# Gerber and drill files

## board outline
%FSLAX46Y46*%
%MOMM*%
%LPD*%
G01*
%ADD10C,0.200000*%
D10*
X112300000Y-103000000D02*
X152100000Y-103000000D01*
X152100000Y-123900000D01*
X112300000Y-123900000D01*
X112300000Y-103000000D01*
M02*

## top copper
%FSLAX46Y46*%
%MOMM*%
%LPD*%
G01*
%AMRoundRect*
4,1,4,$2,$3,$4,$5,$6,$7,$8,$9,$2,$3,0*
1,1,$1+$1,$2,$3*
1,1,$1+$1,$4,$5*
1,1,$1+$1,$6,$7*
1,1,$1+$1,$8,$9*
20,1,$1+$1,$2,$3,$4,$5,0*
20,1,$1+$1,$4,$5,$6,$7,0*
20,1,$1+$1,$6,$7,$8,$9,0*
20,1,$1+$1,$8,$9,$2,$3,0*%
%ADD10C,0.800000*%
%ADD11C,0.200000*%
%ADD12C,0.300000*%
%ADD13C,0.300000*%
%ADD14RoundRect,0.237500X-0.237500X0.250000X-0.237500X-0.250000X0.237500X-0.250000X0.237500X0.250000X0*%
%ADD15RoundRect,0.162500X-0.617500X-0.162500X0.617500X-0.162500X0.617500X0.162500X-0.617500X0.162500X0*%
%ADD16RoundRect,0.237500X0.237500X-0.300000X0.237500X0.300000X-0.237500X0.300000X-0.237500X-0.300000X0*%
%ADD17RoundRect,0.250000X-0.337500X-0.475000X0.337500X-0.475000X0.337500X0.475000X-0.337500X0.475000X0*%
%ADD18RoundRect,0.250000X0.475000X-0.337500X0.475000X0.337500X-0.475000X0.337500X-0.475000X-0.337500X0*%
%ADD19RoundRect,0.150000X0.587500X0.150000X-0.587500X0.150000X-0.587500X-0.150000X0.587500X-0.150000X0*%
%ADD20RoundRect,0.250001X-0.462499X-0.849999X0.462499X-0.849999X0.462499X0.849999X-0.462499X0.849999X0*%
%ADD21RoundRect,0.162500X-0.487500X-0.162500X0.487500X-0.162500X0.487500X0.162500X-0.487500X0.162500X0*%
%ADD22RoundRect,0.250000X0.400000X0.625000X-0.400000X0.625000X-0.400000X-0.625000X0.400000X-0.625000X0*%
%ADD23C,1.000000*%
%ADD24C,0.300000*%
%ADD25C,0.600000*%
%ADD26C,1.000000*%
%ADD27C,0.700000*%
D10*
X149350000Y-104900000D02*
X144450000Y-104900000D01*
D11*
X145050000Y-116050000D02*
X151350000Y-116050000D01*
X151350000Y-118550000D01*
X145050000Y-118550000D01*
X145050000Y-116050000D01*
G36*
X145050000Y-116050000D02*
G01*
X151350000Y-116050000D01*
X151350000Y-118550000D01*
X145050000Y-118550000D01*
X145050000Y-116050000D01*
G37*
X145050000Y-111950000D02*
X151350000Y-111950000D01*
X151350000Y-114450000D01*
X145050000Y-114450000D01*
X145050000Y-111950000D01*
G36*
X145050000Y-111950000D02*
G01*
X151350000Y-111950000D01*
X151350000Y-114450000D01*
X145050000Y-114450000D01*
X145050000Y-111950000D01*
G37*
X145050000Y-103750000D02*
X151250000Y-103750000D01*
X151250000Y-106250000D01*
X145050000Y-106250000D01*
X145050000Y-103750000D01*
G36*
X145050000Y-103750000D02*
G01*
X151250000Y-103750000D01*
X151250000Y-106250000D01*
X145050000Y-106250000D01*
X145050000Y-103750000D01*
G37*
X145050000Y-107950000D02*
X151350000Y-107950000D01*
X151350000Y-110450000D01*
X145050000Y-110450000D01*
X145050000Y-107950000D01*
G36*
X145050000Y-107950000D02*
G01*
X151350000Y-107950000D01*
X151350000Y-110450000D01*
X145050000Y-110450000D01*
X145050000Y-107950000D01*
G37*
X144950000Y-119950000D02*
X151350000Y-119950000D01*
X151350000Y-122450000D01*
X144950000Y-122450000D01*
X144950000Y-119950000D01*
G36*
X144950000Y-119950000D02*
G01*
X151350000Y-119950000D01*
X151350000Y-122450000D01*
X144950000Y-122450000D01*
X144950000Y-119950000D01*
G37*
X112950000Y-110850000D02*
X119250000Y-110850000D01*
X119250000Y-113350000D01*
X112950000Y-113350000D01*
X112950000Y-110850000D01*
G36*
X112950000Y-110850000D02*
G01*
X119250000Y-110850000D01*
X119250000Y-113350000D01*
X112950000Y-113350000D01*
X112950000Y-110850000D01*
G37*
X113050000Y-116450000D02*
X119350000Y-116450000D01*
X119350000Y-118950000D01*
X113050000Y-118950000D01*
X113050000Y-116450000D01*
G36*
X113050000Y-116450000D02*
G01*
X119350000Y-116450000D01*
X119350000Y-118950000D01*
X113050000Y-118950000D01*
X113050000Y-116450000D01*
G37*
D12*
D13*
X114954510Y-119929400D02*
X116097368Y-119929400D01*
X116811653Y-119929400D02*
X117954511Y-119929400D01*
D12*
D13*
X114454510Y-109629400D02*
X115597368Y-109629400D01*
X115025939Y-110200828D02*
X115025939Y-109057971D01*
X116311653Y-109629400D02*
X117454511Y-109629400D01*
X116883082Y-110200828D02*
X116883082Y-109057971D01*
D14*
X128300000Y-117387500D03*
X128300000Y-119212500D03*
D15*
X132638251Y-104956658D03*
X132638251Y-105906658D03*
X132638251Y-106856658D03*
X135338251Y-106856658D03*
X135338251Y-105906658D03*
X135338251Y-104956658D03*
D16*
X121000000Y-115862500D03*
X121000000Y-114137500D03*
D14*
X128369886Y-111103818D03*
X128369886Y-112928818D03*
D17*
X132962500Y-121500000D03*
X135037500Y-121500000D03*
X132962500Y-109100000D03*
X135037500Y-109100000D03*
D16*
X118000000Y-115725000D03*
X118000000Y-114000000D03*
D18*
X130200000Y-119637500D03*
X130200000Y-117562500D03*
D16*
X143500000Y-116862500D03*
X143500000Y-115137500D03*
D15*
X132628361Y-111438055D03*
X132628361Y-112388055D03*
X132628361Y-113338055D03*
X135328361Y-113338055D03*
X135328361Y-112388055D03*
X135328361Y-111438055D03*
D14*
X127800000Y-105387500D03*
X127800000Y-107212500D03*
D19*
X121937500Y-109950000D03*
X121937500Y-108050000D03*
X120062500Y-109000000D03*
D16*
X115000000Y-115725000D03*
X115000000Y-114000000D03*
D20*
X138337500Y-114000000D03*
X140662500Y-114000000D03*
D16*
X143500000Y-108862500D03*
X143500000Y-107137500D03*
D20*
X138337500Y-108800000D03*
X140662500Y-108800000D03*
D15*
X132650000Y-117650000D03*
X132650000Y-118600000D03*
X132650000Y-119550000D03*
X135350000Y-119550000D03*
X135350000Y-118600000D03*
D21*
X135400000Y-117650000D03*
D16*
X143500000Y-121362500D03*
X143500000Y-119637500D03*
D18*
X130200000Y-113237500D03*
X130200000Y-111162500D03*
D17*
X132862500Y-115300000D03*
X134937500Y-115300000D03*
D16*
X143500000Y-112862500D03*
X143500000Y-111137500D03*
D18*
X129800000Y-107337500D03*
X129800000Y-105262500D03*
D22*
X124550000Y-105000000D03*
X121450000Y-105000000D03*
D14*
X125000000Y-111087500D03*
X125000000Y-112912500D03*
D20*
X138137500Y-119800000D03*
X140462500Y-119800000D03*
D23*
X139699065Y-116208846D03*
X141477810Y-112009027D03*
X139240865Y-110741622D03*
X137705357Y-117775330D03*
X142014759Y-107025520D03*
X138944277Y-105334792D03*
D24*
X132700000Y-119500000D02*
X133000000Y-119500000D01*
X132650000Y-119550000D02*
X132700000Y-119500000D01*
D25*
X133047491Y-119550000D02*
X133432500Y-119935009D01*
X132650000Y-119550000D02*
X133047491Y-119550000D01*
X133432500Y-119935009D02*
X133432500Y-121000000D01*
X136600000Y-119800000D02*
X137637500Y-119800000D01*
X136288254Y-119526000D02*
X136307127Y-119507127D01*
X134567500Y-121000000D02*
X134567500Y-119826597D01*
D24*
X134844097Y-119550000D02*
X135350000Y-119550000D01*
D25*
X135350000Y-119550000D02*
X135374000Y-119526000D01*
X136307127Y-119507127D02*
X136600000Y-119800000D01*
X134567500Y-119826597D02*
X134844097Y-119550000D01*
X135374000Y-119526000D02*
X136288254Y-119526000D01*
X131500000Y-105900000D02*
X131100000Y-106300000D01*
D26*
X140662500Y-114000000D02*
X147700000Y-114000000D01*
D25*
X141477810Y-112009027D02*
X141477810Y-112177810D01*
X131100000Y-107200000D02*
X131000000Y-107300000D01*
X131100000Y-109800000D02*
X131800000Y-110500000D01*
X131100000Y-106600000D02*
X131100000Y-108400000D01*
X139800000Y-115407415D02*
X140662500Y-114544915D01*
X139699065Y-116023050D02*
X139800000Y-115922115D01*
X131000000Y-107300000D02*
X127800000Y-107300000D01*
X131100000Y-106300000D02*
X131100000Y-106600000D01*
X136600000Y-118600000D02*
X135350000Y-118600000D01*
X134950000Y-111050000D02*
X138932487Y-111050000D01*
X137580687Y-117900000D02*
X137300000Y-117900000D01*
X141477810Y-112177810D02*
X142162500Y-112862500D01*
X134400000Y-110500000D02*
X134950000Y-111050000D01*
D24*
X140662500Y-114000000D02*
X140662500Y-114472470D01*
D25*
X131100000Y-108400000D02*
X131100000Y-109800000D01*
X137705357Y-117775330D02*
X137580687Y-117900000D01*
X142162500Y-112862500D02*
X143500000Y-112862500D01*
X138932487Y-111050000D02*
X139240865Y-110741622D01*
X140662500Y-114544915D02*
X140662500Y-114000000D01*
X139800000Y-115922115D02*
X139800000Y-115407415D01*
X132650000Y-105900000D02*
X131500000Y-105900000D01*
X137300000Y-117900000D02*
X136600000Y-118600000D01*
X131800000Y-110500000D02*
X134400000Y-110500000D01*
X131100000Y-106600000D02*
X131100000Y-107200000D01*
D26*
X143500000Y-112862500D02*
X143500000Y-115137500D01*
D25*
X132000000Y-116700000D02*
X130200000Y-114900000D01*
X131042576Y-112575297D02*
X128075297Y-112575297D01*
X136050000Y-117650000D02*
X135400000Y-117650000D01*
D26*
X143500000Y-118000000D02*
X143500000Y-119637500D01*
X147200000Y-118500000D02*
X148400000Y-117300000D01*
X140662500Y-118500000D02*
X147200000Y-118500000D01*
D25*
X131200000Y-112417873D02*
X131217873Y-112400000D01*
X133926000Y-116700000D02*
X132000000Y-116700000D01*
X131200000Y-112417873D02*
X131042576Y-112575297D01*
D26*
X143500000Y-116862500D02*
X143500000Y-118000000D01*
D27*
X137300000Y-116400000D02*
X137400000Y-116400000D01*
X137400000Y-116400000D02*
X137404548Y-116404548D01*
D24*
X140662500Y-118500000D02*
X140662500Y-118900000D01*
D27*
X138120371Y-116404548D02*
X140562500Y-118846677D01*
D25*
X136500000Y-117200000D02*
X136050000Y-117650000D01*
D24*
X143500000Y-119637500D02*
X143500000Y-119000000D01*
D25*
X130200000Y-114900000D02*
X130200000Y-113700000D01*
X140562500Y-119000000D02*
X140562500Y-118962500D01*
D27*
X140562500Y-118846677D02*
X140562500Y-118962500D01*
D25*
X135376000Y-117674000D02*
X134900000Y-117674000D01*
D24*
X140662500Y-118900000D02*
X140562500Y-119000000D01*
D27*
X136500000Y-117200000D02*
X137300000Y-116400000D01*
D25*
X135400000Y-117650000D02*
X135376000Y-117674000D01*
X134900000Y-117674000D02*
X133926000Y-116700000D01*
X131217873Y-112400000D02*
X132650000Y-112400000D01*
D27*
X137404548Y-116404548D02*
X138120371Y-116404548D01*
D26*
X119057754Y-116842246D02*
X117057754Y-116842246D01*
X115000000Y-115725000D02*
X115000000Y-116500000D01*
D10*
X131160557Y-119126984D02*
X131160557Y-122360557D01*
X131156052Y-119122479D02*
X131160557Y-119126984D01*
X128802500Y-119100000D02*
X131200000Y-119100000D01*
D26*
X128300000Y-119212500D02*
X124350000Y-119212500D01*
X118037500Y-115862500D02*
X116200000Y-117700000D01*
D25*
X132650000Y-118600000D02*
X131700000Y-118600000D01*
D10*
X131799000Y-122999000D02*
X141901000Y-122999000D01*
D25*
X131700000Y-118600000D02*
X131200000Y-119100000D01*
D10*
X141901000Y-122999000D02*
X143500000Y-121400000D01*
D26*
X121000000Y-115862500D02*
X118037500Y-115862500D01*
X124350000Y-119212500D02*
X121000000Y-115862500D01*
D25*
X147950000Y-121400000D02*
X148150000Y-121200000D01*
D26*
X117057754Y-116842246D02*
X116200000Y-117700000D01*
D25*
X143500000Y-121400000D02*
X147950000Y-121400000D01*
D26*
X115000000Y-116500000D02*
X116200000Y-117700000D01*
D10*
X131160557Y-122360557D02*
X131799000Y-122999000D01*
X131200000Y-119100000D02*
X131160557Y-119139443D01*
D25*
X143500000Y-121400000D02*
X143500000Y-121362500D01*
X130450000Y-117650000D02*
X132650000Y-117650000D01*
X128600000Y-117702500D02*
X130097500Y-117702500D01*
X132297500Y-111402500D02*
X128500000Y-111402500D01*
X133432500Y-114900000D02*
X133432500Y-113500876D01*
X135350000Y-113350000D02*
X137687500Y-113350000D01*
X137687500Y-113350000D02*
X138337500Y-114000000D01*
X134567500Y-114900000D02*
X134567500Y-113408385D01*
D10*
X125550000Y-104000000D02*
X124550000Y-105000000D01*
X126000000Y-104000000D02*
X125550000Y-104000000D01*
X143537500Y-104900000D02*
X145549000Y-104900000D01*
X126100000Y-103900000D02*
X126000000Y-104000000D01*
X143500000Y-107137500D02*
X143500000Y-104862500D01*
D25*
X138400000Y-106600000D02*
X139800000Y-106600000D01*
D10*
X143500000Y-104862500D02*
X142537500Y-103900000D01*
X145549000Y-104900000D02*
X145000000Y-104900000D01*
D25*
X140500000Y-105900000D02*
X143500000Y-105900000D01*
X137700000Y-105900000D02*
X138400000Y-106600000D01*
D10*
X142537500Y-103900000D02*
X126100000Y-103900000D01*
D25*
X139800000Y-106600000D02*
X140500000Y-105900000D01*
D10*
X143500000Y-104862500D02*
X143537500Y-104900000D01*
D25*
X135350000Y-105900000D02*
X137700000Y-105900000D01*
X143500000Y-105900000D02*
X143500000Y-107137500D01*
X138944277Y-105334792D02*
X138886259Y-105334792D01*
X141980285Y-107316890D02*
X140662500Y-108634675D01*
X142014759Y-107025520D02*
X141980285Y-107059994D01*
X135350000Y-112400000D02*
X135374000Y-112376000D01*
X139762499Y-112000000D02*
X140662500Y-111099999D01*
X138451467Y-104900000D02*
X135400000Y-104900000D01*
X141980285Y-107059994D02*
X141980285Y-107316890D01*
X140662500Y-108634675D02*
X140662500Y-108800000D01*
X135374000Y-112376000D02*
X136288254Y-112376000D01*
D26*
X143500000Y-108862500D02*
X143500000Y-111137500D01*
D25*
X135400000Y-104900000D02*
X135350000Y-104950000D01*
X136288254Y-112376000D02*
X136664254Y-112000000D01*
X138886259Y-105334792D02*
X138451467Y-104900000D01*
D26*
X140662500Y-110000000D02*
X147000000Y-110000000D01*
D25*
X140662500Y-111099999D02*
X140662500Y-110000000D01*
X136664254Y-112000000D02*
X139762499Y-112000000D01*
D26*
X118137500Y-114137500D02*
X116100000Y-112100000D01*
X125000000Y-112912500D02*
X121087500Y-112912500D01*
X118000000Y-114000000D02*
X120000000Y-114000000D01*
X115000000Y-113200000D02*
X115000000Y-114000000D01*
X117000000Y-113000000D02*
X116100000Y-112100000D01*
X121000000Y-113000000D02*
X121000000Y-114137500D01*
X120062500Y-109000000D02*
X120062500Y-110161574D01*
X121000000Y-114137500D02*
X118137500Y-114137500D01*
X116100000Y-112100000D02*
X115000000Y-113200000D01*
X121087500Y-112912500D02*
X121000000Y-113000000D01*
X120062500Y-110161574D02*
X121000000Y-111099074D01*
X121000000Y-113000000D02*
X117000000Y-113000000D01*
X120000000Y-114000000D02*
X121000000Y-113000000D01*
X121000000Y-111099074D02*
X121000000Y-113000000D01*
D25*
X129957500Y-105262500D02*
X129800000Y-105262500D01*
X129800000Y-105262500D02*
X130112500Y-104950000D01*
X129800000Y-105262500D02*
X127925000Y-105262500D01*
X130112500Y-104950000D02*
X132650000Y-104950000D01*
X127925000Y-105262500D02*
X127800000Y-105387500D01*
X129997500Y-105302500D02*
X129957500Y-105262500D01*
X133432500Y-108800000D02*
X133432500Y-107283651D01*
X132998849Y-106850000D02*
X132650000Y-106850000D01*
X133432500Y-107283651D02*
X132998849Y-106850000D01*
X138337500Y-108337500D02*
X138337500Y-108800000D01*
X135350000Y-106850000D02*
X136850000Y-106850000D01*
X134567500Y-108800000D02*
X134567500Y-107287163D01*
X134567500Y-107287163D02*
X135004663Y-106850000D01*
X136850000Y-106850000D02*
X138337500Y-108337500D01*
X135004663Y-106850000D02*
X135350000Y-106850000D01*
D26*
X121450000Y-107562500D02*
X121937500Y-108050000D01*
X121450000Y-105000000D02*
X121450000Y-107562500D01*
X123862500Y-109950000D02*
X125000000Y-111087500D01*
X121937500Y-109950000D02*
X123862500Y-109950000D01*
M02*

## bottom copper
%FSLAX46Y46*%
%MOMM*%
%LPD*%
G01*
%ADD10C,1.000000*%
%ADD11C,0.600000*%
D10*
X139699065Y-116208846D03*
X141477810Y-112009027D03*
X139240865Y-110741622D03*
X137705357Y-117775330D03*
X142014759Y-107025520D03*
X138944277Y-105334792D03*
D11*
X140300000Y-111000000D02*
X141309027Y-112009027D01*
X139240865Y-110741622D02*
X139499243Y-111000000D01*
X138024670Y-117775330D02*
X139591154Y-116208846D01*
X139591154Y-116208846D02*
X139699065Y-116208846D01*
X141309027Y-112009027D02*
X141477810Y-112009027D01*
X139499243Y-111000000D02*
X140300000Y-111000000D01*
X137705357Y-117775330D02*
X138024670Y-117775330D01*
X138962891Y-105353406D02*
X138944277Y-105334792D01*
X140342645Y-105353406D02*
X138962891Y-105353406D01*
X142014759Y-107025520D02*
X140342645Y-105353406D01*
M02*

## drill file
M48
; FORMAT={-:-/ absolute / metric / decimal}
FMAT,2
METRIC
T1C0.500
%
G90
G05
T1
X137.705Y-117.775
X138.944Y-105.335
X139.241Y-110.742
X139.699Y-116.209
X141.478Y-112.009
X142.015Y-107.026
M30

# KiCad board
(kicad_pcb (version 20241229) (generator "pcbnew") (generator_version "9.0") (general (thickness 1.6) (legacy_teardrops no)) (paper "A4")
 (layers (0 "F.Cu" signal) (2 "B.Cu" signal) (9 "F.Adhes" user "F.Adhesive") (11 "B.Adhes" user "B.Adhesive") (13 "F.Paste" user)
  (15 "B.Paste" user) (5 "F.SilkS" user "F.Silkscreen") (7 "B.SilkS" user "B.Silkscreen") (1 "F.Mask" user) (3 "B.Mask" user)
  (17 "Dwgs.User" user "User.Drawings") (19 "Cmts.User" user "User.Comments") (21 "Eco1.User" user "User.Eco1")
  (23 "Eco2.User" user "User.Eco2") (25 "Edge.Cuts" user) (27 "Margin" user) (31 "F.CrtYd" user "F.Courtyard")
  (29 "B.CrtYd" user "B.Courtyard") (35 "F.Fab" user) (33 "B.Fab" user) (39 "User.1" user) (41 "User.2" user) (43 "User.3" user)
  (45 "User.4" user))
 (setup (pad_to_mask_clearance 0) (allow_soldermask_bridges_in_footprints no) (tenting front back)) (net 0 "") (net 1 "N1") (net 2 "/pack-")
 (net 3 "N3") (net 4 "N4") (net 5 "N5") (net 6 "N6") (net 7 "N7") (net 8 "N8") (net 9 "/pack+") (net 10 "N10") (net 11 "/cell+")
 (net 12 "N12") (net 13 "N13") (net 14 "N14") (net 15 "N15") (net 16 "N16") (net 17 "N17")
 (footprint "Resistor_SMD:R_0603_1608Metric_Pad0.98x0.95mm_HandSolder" (layer "F.Cu") (at 128.3 118.3 -90)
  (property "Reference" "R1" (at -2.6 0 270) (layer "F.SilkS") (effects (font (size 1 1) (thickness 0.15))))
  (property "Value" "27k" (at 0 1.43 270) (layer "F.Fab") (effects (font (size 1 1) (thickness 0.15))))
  (pad "1" smd roundrect (at -0.9125 0 270) (size 0.975 0.95) (layers "F.Cu" "F.Mask" "F.Paste") (roundrect_rratio 0.25) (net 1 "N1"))
  (pad "2" smd roundrect (at 0.9125 0 270) (size 0.975 0.95) (layers "F.Cu" "F.Mask" "F.Paste") (roundrect_rratio 0.25) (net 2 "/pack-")))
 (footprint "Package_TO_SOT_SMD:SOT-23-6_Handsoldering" (layer "F.Cu") (at 133.988251 105.906658)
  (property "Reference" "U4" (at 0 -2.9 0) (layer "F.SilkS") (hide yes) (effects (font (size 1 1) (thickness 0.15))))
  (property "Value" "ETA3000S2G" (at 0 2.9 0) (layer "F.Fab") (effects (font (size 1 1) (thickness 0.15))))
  (pad "1" smd roundrect (at -1.35 -0.95) (size 1.56 0.65) (layers "F.Cu" "F.Mask" "F.Paste") (roundrect_rratio 0.25) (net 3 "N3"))
  (pad "2" smd roundrect (at -1.35 0) (size 1.56 0.65) (layers "F.Cu" "F.Mask" "F.Paste") (roundrect_rratio 0.25) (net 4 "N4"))
  (pad "3" smd roundrect (at -1.35 0.95) (size 1.56 0.65) (layers "F.Cu" "F.Mask" "F.Paste") (roundrect_rratio 0.25) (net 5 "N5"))
  (pad "4" smd roundrect (at 1.35 0.95) (size 1.56 0.65) (layers "F.Cu" "F.Mask" "F.Paste") (roundrect_rratio 0.25) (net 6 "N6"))
  (pad "5" smd roundrect (at 1.35 0) (size 1.56 0.65) (layers "F.Cu" "F.Mask" "F.Paste") (roundrect_rratio 0.25) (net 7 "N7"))
  (pad "6" smd roundrect (at 1.35 -0.95) (size 1.56 0.65) (layers "F.Cu" "F.Mask" "F.Paste") (roundrect_rratio 0.25) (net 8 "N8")))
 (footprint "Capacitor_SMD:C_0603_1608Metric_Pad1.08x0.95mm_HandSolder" (layer "F.Cu") (at 121 115 90)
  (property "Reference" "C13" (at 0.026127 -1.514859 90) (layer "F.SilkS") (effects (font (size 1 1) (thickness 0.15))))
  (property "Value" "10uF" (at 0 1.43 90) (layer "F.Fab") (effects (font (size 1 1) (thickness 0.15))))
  (pad "1" smd roundrect (at -0.8625 0 90) (size 1.075 0.95) (layers "F.Cu" "F.Mask" "F.Paste") (roundrect_rratio 0.25) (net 2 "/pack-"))
  (pad "2" smd roundrect (at 0.8625 0 90) (size 1.075 0.95) (layers "F.Cu" "F.Mask" "F.Paste") (roundrect_rratio 0.25) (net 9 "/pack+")))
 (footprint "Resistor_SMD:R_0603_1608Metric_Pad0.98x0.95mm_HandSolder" (layer "F.Cu") (at 128.369886 112.016318 -90)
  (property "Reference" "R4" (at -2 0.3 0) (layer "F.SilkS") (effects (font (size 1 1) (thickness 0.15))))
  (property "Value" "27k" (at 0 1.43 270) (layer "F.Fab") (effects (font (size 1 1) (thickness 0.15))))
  (pad "1" smd roundrect (at -0.9125 0 270) (size 0.975 0.95) (layers "F.Cu" "F.Mask" "F.Paste") (roundrect_rratio 0.25) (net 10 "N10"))
  (pad "2" smd roundrect (at 0.9125 0 270) (size 0.975 0.95) (layers "F.Cu" "F.Mask" "F.Paste") (roundrect_rratio 0.25) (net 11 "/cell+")))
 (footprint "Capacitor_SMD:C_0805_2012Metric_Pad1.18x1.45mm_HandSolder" (layer "F.Cu") (at 134 121.5)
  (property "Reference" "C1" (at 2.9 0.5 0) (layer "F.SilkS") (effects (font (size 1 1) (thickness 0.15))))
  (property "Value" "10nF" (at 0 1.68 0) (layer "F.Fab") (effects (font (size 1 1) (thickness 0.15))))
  (pad "1" smd roundrect (at -1.0375 0) (size 1.175 1.45) (layers "F.Cu" "F.Mask" "F.Paste") (roundrect_rratio 0.212766) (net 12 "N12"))
  (pad "2" smd roundrect (at 1.0375 0) (size 1.175 1.45) (layers "F.Cu" "F.Mask" "F.Paste") (roundrect_rratio 0.212766) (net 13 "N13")))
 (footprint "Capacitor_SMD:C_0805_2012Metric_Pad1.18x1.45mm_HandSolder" (layer "F.Cu") (at 134 109.1)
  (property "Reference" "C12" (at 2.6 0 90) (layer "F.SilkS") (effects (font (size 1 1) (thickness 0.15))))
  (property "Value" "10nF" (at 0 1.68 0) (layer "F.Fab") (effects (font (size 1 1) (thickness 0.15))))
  (pad "1" smd roundrect (at -1.0375 0) (size 1.175 1.45) (layers "F.Cu" "F.Mask" "F.Paste") (roundrect_rratio 0.212766) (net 5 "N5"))
  (pad "2" smd roundrect (at 1.0375 0) (size 1.175 1.45) (layers "F.Cu" "F.Mask" "F.Paste") (roundrect_rratio 0.212766) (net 6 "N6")))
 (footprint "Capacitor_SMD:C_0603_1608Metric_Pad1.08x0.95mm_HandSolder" (layer "F.Cu") (at 118 114.8625 90)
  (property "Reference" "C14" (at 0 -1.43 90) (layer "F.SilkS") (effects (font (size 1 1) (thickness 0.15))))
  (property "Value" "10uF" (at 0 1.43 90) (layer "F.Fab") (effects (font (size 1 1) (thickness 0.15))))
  (pad "1" smd roundrect (at -0.8625 0 90) (size 1.075 0.95) (layers "F.Cu" "F.Mask" "F.Paste") (roundrect_rratio 0.25) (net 2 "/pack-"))
  (pad "2" smd roundrect (at 0.8625 0 90) (size 1.075 0.95) (layers "F.Cu" "F.Mask" "F.Paste") (roundrect_rratio 0.25) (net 9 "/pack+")))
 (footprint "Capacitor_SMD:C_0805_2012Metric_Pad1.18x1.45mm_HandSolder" (layer "F.Cu") (at 130.2 118.6 90)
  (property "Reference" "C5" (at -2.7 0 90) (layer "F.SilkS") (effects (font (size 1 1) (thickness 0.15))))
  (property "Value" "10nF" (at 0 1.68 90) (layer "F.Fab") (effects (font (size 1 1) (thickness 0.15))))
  (pad "1" smd roundrect (at -1.0375 0 90) (size 1.175 1.45) (layers "F.Cu" "F.Mask" "F.Paste") (roundrect_rratio 0.212766) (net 2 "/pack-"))
  (pad "2" smd roundrect (at 1.0375 0 90) (size 1.175 1.45) (layers "F.Cu" "F.Mask" "F.Paste") (roundrect_rratio 0.212766) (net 1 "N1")))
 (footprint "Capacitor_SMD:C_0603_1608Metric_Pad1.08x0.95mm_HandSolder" (layer "F.Cu") (at 143.5 116 90)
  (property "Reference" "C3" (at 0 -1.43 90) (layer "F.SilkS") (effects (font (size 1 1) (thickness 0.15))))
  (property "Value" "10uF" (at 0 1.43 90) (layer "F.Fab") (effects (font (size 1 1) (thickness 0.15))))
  (pad "1" smd roundrect (at -0.8625 0 90) (size 1.075 0.95) (layers "F.Cu" "F.Mask" "F.Paste") (roundrect_rratio 0.25) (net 11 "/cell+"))
  (pad "2" smd roundrect (at 0.8625 0 90) (size 1.075 0.95) (layers "F.Cu" "F.Mask" "F.Paste") (roundrect_rratio 0.25) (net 4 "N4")))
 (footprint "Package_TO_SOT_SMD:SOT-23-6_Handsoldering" (layer "F.Cu") (at 133.978361 112.388055)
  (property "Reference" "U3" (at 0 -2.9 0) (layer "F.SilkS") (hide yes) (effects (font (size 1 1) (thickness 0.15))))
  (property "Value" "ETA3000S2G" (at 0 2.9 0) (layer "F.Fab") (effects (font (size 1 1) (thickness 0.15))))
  (pad "1" smd roundrect (at -1.35 -0.95) (size 1.56 0.65) (layers "F.Cu" "F.Mask" "F.Paste") (roundrect_rratio 0.25) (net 10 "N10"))
  (pad "2" smd roundrect (at -1.35 0) (size 1.56 0.65) (layers "F.Cu" "F.Mask" "F.Paste") (roundrect_rratio 0.25) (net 11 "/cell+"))
  (pad "3" smd roundrect (at -1.35 0.95) (size 1.56 0.65) (layers "F.Cu" "F.Mask" "F.Paste") (roundrect_rratio 0.25) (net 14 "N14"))
  (pad "4" smd roundrect (at 1.35 0.95) (size 1.56 0.65) (layers "F.Cu" "F.Mask" "F.Paste") (roundrect_rratio 0.25) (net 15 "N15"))
  (pad "5" smd roundrect (at 1.35 0) (size 1.56 0.65) (layers "F.Cu" "F.Mask" "F.Paste") (roundrect_rratio 0.25) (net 8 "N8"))
  (pad "6" smd roundrect (at 1.35 -0.95) (size 1.56 0.65) (layers "F.Cu" "F.Mask" "F.Paste") (roundrect_rratio 0.25) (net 4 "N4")))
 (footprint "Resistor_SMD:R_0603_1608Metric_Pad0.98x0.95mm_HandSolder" (layer "F.Cu") (at 127.8 106.3 -90)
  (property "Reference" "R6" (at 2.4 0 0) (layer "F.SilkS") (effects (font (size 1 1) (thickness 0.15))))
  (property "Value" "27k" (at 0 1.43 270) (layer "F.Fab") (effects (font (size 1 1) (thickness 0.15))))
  (pad "1" smd roundrect (at -0.9125 0 270) (size 0.975 0.95) (layers "F.Cu" "F.Mask" "F.Paste") (roundrect_rratio 0.25) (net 3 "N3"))
  (pad "2" smd roundrect (at 0.9125 0 270) (size 0.975 0.95) (layers "F.Cu" "F.Mask" "F.Paste") (roundrect_rratio 0.25) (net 4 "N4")))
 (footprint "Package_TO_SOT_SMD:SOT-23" (layer "F.Cu") (at 121 109 180)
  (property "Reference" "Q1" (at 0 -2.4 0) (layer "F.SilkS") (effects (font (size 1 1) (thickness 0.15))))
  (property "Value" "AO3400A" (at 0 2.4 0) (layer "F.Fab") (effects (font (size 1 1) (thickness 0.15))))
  (pad "1" smd roundrect (at -0.9375 -0.95 180) (size 1.475 0.6) (layers "F.Cu" "F.Mask" "F.Paste") (roundrect_rratio 0.25) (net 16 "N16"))
  (pad "2" smd roundrect (at -0.9375 0.95 180) (size 1.475 0.6) (layers "F.Cu" "F.Mask" "F.Paste") (roundrect_rratio 0.25) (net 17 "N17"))
  (pad "3" smd roundrect (at 0.9375 0 180) (size 1.475 0.6) (layers "F.Cu" "F.Mask" "F.Paste") (roundrect_rratio 0.25) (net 9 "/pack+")))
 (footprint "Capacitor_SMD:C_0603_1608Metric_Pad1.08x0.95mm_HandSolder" (layer "F.Cu") (at 115 114.8625 90)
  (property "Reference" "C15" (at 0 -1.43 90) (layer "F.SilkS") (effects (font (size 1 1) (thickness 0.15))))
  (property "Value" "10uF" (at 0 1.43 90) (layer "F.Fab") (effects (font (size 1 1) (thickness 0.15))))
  (pad "1" smd roundrect (at -0.8625 0 90) (size 1.075 0.95) (layers "F.Cu" "F.Mask" "F.Paste") (roundrect_rratio 0.25) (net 2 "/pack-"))
  (pad "2" smd roundrect (at 0.8625 0 90) (size 1.075 0.95) (layers "F.Cu" "F.Mask" "F.Paste") (roundrect_rratio 0.25) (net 9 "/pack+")))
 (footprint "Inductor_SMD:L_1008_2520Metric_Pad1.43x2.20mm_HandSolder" (layer "F.Cu") (at 139.5 114)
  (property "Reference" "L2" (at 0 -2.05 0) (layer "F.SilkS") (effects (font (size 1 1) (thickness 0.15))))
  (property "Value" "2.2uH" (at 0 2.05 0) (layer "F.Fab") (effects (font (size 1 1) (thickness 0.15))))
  (pad "1" smd roundrect (at -1.1625 0) (size 1.425 2.2) (layers "F.Cu" "F.Mask" "F.Paste") (roundrect_rratio 0.175439) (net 15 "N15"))
  (pad "2" smd roundrect (at 1.1625 0) (size 1.425 2.2) (layers "F.Cu" "F.Mask" "F.Paste") (roundrect_rratio 0.175439) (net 4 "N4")))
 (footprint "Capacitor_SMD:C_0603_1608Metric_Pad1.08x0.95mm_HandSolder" (layer "F.Cu") (at 143.5 108 90)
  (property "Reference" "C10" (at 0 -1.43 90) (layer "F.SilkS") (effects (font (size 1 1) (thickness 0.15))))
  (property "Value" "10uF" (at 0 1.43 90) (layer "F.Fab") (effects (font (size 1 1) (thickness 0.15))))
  (pad "1" smd roundrect (at -0.8625 0 90) (size 1.075 0.95) (layers "F.Cu" "F.Mask" "F.Paste") (roundrect_rratio 0.25) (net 8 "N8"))
  (pad "2" smd roundrect (at 0.8625 0 90) (size 1.075 0.95) (layers "F.Cu" "F.Mask" "F.Paste") (roundrect_rratio 0.25) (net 7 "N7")))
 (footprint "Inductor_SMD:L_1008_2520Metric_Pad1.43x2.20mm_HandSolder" (layer "F.Cu") (at 139.5 108.8)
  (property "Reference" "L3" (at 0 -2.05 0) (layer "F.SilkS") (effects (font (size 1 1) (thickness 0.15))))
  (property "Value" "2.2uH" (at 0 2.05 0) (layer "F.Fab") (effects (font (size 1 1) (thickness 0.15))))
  (pad "1" smd roundrect (at -1.1625 0) (size 1.425 2.2) (layers "F.Cu" "F.Mask" "F.Paste") (roundrect_rratio 0.175439) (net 6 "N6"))
  (pad "2" smd roundrect (at 1.1625 0) (size 1.425 2.2) (layers "F.Cu" "F.Mask" "F.Paste") (roundrect_rratio 0.175439) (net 8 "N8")))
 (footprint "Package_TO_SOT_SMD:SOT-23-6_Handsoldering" (layer "F.Cu") (at 134 118.6)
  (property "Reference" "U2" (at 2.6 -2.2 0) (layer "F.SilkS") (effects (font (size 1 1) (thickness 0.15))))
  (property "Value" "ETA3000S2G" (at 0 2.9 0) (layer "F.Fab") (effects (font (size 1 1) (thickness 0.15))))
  (pad "1" smd roundrect (at -1.35 -0.95) (size 1.56 0.65) (layers "F.Cu" "F.Mask" "F.Paste") (roundrect_rratio 0.25) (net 1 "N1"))
  (pad "2" smd roundrect (at -1.35 0) (size 1.56 0.65) (layers "F.Cu" "F.Mask" "F.Paste") (roundrect_rratio 0.25) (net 2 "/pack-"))
  (pad "3" smd roundrect (at -1.35 0.95) (size 1.56 0.65) (layers "F.Cu" "F.Mask" "F.Paste") (roundrect_rratio 0.25) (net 12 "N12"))
  (pad "4" smd roundrect (at 1.35 0.95) (size 1.56 0.65) (layers "F.Cu" "F.Mask" "F.Paste") (roundrect_rratio 0.25) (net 13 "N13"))
  (pad "5" smd roundrect (at 1.35 0) (size 1.56 0.65) (layers "F.Cu" "F.Mask" "F.Paste") (roundrect_rratio 0.25) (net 4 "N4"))
  (pad "6" smd roundrect (at 1.4 -0.95) (size 1.3 0.65) (layers "F.Cu" "F.Mask" "F.Paste") (roundrect_rratio 0.25) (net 11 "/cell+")))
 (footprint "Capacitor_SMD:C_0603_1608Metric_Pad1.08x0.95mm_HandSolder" (layer "F.Cu") (at 143.5 120.5 90)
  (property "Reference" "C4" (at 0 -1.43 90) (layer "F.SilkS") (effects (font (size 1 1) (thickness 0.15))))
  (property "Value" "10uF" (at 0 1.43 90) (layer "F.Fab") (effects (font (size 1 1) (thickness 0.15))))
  (pad "1" smd roundrect (at -0.8625 0 90) (size 1.075 0.95) (layers "F.Cu" "F.Mask" "F.Paste") (roundrect_rratio 0.25) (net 2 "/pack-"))
  (pad "2" smd roundrect (at 0.8625 0 90) (size 1.075 0.95) (layers "F.Cu" "F.Mask" "F.Paste") (roundrect_rratio 0.25) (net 11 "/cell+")))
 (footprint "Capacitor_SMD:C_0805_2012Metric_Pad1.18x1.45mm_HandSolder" (layer "F.Cu") (at 130.2 112.2 90)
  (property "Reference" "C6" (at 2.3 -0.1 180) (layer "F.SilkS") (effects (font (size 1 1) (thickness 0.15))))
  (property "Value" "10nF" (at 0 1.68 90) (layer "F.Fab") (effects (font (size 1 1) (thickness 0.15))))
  (pad "1" smd roundrect (at -1.0375 0 90) (size 1.175 1.45) (layers "F.Cu" "F.Mask" "F.Paste") (roundrect_rratio 0.212766)
   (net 11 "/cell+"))
  (pad "2" smd roundrect (at 1.0375 0 90) (size 1.175 1.45) (layers "F.Cu" "F.Mask" "F.Paste") (roundrect_rratio 0.212766) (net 10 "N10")))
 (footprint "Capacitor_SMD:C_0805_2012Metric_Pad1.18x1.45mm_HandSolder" (layer "F.Cu") (at 133.9 115.3)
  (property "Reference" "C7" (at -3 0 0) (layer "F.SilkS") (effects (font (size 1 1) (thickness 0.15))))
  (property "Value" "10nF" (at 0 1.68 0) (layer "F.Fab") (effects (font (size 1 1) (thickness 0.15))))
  (pad "1" smd roundrect (at -1.0375 0) (size 1.175 1.45) (layers "F.Cu" "F.Mask" "F.Paste") (roundrect_rratio 0.212766) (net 14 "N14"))
  (pad "2" smd roundrect (at 1.0375 0) (size 1.175 1.45) (layers "F.Cu" "F.Mask" "F.Paste") (roundrect_rratio 0.212766) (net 15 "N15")))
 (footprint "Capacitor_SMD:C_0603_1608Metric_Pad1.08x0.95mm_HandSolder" (layer "F.Cu") (at 143.5 112 90)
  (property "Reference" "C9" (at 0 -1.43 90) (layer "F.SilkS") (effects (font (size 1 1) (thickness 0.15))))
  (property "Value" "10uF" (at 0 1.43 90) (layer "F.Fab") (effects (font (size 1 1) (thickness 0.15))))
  (pad "1" smd roundrect (at -0.8625 0 90) (size 1.075 0.95) (layers "F.Cu" "F.Mask" "F.Paste") (roundrect_rratio 0.25) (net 4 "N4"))
  (pad "2" smd roundrect (at 0.8625 0 90) (size 1.075 0.95) (layers "F.Cu" "F.Mask" "F.Paste") (roundrect_rratio 0.25) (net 8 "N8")))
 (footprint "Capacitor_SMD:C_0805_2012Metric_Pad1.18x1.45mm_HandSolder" (layer "F.Cu") (at 129.8 106.3 90)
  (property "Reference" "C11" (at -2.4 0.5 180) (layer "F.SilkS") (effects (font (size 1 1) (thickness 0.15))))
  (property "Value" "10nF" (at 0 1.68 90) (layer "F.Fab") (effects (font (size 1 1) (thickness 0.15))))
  (pad "1" smd roundrect (at -1.0375 0 90) (size 1.175 1.45) (layers "F.Cu" "F.Mask" "F.Paste") (roundrect_rratio 0.212766) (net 4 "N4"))
  (pad "2" smd roundrect (at 1.0375 0 90) (size 1.175 1.45) (layers "F.Cu" "F.Mask" "F.Paste") (roundrect_rratio 0.212766) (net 3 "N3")))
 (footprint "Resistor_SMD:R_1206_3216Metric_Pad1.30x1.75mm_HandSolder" (layer "F.Cu") (at 123 105 180)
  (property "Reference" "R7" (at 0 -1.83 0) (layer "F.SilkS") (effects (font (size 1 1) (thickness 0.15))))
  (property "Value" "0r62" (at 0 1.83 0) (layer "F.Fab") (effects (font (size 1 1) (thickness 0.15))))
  (pad "1" smd roundrect (at -1.55 0 180) (size 1.3 1.75) (layers "F.Cu" "F.Mask" "F.Paste") (roundrect_rratio 0.192308) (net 7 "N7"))
  (pad "2" smd roundrect (at 1.55 0 180) (size 1.3 1.75) (layers "F.Cu" "F.Mask" "F.Paste") (roundrect_rratio 0.192308) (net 17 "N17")))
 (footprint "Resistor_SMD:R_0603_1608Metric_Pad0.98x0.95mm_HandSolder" (layer "F.Cu") (at 125 112 -90)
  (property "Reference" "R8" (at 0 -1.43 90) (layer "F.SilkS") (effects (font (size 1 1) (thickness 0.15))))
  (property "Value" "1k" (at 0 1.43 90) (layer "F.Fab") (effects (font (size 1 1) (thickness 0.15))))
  (pad "1" smd roundrect (at -0.9125 0 270) (size 0.975 0.95) (layers "F.Cu" "F.Mask" "F.Paste") (roundrect_rratio 0.25) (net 16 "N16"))
  (pad "2" smd roundrect (at 0.9125 0 270) (size 0.975 0.95) (layers "F.Cu" "F.Mask" "F.Paste") (roundrect_rratio 0.25) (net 9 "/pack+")))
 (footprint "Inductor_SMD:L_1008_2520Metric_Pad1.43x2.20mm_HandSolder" (layer "F.Cu") (at 139.3 119.8)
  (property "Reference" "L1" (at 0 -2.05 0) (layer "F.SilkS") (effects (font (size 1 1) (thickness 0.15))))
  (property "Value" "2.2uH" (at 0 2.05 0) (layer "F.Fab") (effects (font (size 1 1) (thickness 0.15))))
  (pad "1" smd roundrect (at -1.1625 0) (size 1.425 2.2) (layers "F.Cu" "F.Mask" "F.Paste") (roundrect_rratio 0.175439) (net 13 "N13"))
  (pad "2" smd roundrect (at 1.1625 0) (size 1.425 2.2) (layers "F.Cu" "F.Mask" "F.Paste") (roundrect_rratio 0.175439) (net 11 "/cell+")))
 (gr_line (start 149.35 104.9) (end 144.45 104.9) (stroke (width 0.8) (type solid)) (layer "F.Cu") (net 7))
 (gr_rect (start 145.05 116.05) (end 151.35 118.55) (stroke (width 0.2) (type solid)) (fill yes) (layers "F.Cu" "F.Mask")
  (solder_mask_margin 0) (net 11))
 (gr_rect (start 145.05 111.95) (end 151.35 114.45) (stroke (width 0.2) (type solid)) (fill yes) (layers "F.Cu" "F.Mask")
  (solder_mask_margin 0) (net 4))
 (gr_rect (start 145.05 103.75) (end 151.25 106.25) (stroke (width 0.2) (type solid)) (fill yes) (layers "F.Cu" "F.Mask")
  (solder_mask_margin 0) (net 7))
 (gr_rect (start 145.05 107.95) (end 151.35 110.45) (stroke (width 0.2) (type solid)) (fill yes) (layers "F.Cu" "F.Mask")
  (solder_mask_margin 0) (net 8))
 (gr_rect (start 144.95 119.95) (end 151.35 122.45) (stroke (width 0.2) (type solid)) (fill yes) (layers "F.Cu" "F.Mask")
  (solder_mask_margin 0) (net 2))
 (gr_rect (start 112.95 110.85) (end 119.25 113.35) (stroke (width 0.2) (type solid)) (fill yes) (layers "F.Cu" "F.Mask")
  (solder_mask_margin 0) (net 9))
 (gr_rect (start 113.05 116.45) (end 119.35 118.95) (stroke (width 0.2) (type solid)) (fill yes) (layers "F.Cu" "F.Mask")
  (solder_mask_margin 0) (net 2))
 (gr_rect (start 112.3 103) (end 152.1 123.9) (stroke (width 0.2) (type solid)) (fill no) (layer "Edge.Cuts"))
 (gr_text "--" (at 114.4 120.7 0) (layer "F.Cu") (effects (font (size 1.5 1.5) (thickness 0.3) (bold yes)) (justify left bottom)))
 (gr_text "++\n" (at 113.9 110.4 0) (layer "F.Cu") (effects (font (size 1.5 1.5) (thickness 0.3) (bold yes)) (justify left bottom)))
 (segment (start 132.7 119.5) (end 133 119.5) (width 0.3) (layer "F.Cu") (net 12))
 (segment (start 132.65 119.55) (end 132.7 119.5) (width 0.3) (layer "F.Cu") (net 12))
 (segment (start 133.047491 119.55) (end 133.4325 119.935009) (width 0.6) (layer "F.Cu") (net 12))
 (segment (start 132.65 119.55) (end 133.047491 119.55) (width 0.6) (layer "F.Cu") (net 12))
 (segment (start 133.4325 119.935009) (end 133.4325 121) (width 0.6) (layer "F.Cu") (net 12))
 (segment (start 136.6 119.8) (end 137.6375 119.8) (width 0.6) (layer "F.Cu") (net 13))
 (segment (start 136.288254 119.526) (end 136.307127 119.507127) (width 0.6) (layer "F.Cu") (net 13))
 (segment (start 134.5675 121) (end 134.5675 119.826597) (width 0.6) (layer "F.Cu") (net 13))
 (segment (start 134.844097 119.55) (end 135.35 119.55) (width 0.3) (layer "F.Cu") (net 13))
 (segment (start 135.35 119.55) (end 135.374 119.526) (width 0.6) (layer "F.Cu") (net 13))
 (segment (start 136.307127 119.507127) (end 136.6 119.8) (width 0.6) (layer "F.Cu") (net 13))
 (segment (start 134.5675 119.826597) (end 134.844097 119.55) (width 0.6) (layer "F.Cu") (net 13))
 (segment (start 135.374 119.526) (end 136.288254 119.526) (width 0.6) (layer "F.Cu") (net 13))
 (segment (start 131.5 105.9) (end 131.1 106.3) (width 0.6) (layer "F.Cu") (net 4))
 (segment (start 140.6625 114) (end 147.7 114) (width 1) (layer "F.Cu") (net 4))
 (segment (start 141.47781 112.009027) (end 141.47781 112.17781) (width 0.6) (layer "F.Cu") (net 4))
 (segment (start 131.1 107.2) (end 131 107.3) (width 0.6) (layer "F.Cu") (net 4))
 (segment (start 131.1 109.8) (end 131.8 110.5) (width 0.6) (layer "F.Cu") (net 4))
 (segment (start 131.1 106.6) (end 131.1 108.4) (width 0.6) (layer "F.Cu") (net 4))
 (segment (start 139.8 115.407415) (end 140.6625 114.544915) (width 0.6) (layer "F.Cu") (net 4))
 (segment (start 139.699065 116.02305) (end 139.8 115.922115) (width 0.6) (layer "F.Cu") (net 4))
 (segment (start 131 107.3) (end 127.8 107.3) (width 0.6) (layer "F.Cu") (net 4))
 (segment (start 131.1 106.3) (end 131.1 106.6) (width 0.6) (layer "F.Cu") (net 4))
 (segment (start 136.6 118.6) (end 135.35 118.6) (width 0.6) (layer "F.Cu") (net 4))
 (segment (start 134.95 111.05) (end 138.932487 111.05) (width 0.6) (layer "F.Cu") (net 4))
 (segment (start 137.580687 117.9) (end 137.3 117.9) (width 0.6) (layer "F.Cu") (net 4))
 (segment (start 141.47781 112.17781) (end 142.1625 112.8625) (width 0.6) (layer "F.Cu") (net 4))
 (segment (start 134.4 110.5) (end 134.95 111.05) (width 0.6) (layer "F.Cu") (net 4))
 (segment (start 140.6625 114) (end 140.6625 114.47247) (width 0.3) (layer "F.Cu") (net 4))
 (segment (start 131.1 108.4) (end 131.1 109.8) (width 0.6) (layer "F.Cu") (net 4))
 (segment (start 137.705357 117.77533) (end 137.580687 117.9) (width 0.6) (layer "F.Cu") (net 4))
 (segment (start 142.1625 112.8625) (end 143.5 112.8625) (width 0.6) (layer "F.Cu") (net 4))
 (segment (start 138.932487 111.05) (end 139.240865 110.741622) (width 0.6) (layer "F.Cu") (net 4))
 (segment (start 140.6625 114.544915) (end 140.6625 114) (width 0.6) (layer "F.Cu") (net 4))
 (segment (start 139.8 115.922115) (end 139.8 115.407415) (width 0.6) (layer "F.Cu") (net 4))
 (segment (start 132.65 105.9) (end 131.5 105.9) (width 0.6) (layer "F.Cu") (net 4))
 (segment (start 137.3 117.9) (end 136.6 118.6) (width 0.6) (layer "F.Cu") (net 4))
 (segment (start 131.8 110.5) (end 134.4 110.5) (width 0.6) (layer "F.Cu") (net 4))
 (segment (start 131.1 106.6) (end 131.1 107.2) (width 0.6) (layer "F.Cu") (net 4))
 (segment (start 143.5 112.8625) (end 143.5 115.1375) (width 1) (layer "F.Cu") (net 4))
 (via (at 139.699065 116.208846) (size 1) (drill 0.5) (layers "F.Cu" "B.Cu") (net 4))
 (via (at 141.47781 112.009027) (size 1) (drill 0.5) (layers "F.Cu" "B.Cu") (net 4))
 (via (at 139.240865 110.741622) (size 1) (drill 0.5) (layers "F.Cu" "B.Cu") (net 4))
 (via (at 137.705357 117.77533) (size 1) (drill 0.5) (layers "F.Cu" "B.Cu") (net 4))
 (segment (start 140.3 111) (end 141.309027 112.009027) (width 0.6) (layer "B.Cu") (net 4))
 (segment (start 139.240865 110.741622) (end 139.499243 111) (width 0.6) (layer "B.Cu") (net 4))
 (segment (start 138.02467 117.77533) (end 139.591154 116.208846) (width 0.6) (layer "B.Cu") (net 4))
 (segment (start 139.591154 116.208846) (end 139.699065 116.208846) (width 0.6) (layer "B.Cu") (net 4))
 (segment (start 141.309027 112.009027) (end 141.47781 112.009027) (width 0.6) (layer "B.Cu") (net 4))
 (segment (start 139.499243 111) (end 140.3 111) (width 0.6) (layer "B.Cu") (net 4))
 (segment (start 137.705357 117.77533) (end 138.02467 117.77533) (width 0.6) (layer "B.Cu") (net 4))
 (segment (start 132 116.7) (end 130.2 114.9) (width 0.6) (layer "F.Cu") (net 11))
 (segment (start 131.042576 112.575297) (end 128.075297 112.575297) (width 0.6) (layer "F.Cu") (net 11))
 (segment (start 136.05 117.65) (end 135.4 117.65) (width 0.6) (layer "F.Cu") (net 11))
 (segment (start 143.5 118) (end 143.5 119.6375) (width 1) (layer "F.Cu") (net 11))
 (segment (start 147.2 118.5) (end 148.4 117.3) (width 1) (layer "F.Cu") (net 11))
 (segment (start 140.6625 118.5) (end 147.2 118.5) (width 1) (layer "F.Cu") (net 11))
 (segment (start 131.2 112.417873) (end 131.217873 112.4) (width 0.6) (layer "F.Cu") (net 11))
 (segment (start 133.926 116.7) (end 132 116.7) (width 0.6) (layer "F.Cu") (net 11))
 (segment (start 131.2 112.417873) (end 131.042576 112.575297) (width 0.6) (layer "F.Cu") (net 11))
 (segment (start 143.5 116.8625) (end 143.5 118) (width 1) (layer "F.Cu") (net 11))
 (segment (start 137.3 116.4) (end 137.4 116.4) (width 0.7) (layer "F.Cu") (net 11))
 (segment (start 137.4 116.4) (end 137.404548 116.404548) (width 0.7) (layer "F.Cu") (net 11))
 (segment (start 140.6625 118.5) (end 140.6625 118.9) (width 0.3) (layer "F.Cu") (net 11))
 (segment (start 138.120371 116.404548) (end 140.5625 118.846677) (width 0.7) (layer "F.Cu") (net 11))
 (segment (start 136.5 117.2) (end 136.05 117.65) (width 0.6) (layer "F.Cu") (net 11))
 (segment (start 143.5 119.6375) (end 143.5 119) (width 0.3) (layer "F.Cu") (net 11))
 (segment (start 130.2 114.9) (end 130.2 113.7) (width 0.6) (layer "F.Cu") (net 11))
 (segment (start 140.5625 119) (end 140.5625 118.9625) (width 0.6) (layer "F.Cu") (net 11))
 (segment (start 140.5625 118.846677) (end 140.5625 118.9625) (width 0.7) (layer "F.Cu") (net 11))
 (segment (start 135.376 117.674) (end 134.9 117.674) (width 0.6) (layer "F.Cu") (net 11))
 (segment (start 140.6625 118.9) (end 140.5625 119) (width 0.3) (layer "F.Cu") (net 11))
 (segment (start 136.5 117.2) (end 137.3 116.4) (width 0.7) (layer "F.Cu") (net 11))
 (segment (start 135.4 117.65) (end 135.376 117.674) (width 0.6) (layer "F.Cu") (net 11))
 (segment (start 134.9 117.674) (end 133.926 116.7) (width 0.6) (layer "F.Cu") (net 11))
 (segment (start 131.217873 112.4) (end 132.65 112.4) (width 0.6) (layer "F.Cu") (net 11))
 (segment (start 137.404548 116.404548) (end 138.120371 116.404548) (width 0.7) (layer "F.Cu") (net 11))
 (segment (start 119.057754 116.842246) (end 117.057754 116.842246) (width 1) (layer "F.Cu") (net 2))
 (segment (start 115 115.725) (end 115 116.5) (width 1) (layer "F.Cu") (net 2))
 (segment (start 131.160557 119.126984) (end 131.160557 122.360557) (width 0.8) (layer "F.Cu") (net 2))
 (segment (start 131.156052 119.122479) (end 131.160557 119.126984) (width 0.8) (layer "F.Cu") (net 2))
 (segment (start 128.8025 119.1) (end 131.2 119.1) (width 0.8) (layer "F.Cu") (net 2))
 (segment (start 128.3 119.2125) (end 124.35 119.2125) (width 1) (layer "F.Cu") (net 2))
 (segment (start 118.0375 115.8625) (end 116.2 117.7) (width 1) (layer "F.Cu") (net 2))
 (segment (start 132.65 118.6) (end 131.7 118.6) (width 0.6) (layer "F.Cu") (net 2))
 (segment (start 131.799 122.999) (end 141.901 122.999) (width 0.8) (layer "F.Cu") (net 2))
 (segment (start 131.7 118.6) (end 131.2 119.1) (width 0.6) (layer "F.Cu") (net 2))
 (segment (start 141.901 122.999) (end 143.5 121.4) (width 0.8) (layer "F.Cu") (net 2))
 (segment (start 121 115.8625) (end 118.0375 115.8625) (width 1) (layer "F.Cu") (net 2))
 (segment (start 124.35 119.2125) (end 121 115.8625) (width 1) (layer "F.Cu") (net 2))
 (segment (start 147.95 121.4) (end 148.15 121.2) (width 0.6) (layer "F.Cu") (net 2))
 (segment (start 117.057754 116.842246) (end 116.2 117.7) (width 1) (layer "F.Cu") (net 2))
 (segment (start 143.5 121.4) (end 147.95 121.4) (width 0.6) (layer "F.Cu") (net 2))
 (segment (start 115 116.5) (end 116.2 117.7) (width 1) (layer "F.Cu") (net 2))
 (segment (start 131.160557 122.360557) (end 131.799 122.999) (width 0.8) (layer "F.Cu") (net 2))
 (segment (start 131.2 119.1) (end 131.160557 119.139443) (width 0.8) (layer "F.Cu") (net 2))
 (segment (start 143.5 121.4) (end 143.5 121.3625) (width 0.6) (layer "F.Cu") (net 2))
 (segment (start 130.45 117.65) (end 132.65 117.65) (width 0.6) (layer "F.Cu") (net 1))
 (segment (start 128.6 117.7025) (end 130.0975 117.7025) (width 0.6) (layer "F.Cu") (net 1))
 (segment (start 132.2975 111.4025) (end 128.5 111.4025) (width 0.6) (layer "F.Cu") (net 10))
 (segment (start 133.4325 114.9) (end 133.4325 113.500876) (width 0.6) (layer "F.Cu") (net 14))
 (segment (start 135.35 113.35) (end 137.6875 113.35) (width 0.6) (layer "F.Cu") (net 15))
 (segment (start 137.6875 113.35) (end 138.3375 114) (width 0.6) (layer "F.Cu") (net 15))
 (segment (start 134.5675 114.9) (end 134.5675 113.408385) (width 0.6) (layer "F.Cu") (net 15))
 (segment (start 125.55 104) (end 124.55 105) (width 0.8) (layer "F.Cu") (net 7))
 (segment (start 126 104) (end 125.55 104) (width 0.8) (layer "F.Cu") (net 7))
 (segment (start 143.5375 104.9) (end 145.549 104.9) (width 0.8) (layer "F.Cu") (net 7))
 (segment (start 126.1 103.9) (end 126 104) (width 0.8) (layer "F.Cu") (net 7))
 (segment (start 143.5 107.1375) (end 143.5 104.8625) (width 0.8) (layer "F.Cu") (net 7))
 (segment (start 138.4 106.6) (end 139.8 106.6) (width 0.6) (layer "F.Cu") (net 7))
 (segment (start 143.5 104.8625) (end 142.5375 103.9) (width 0.8) (layer "F.Cu") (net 7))
 (segment (start 145.549 104.9) (end 145 104.9) (width 0.8) (layer "F.Cu") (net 7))
 (segment (start 140.5 105.9) (end 143.5 105.9) (width 0.6) (layer "F.Cu") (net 7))
 (segment (start 137.7 105.9) (end 138.4 106.6) (width 0.6) (layer "F.Cu") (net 7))
 (segment (start 142.5375 103.9) (end 126.1 103.9) (width 0.8) (layer "F.Cu") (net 7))
 (segment (start 139.8 106.6) (end 140.5 105.9) (width 0.6) (layer "F.Cu") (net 7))
 (segment (start 143.5 104.8625) (end 143.5375 104.9) (width 0.8) (layer "F.Cu") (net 7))
 (segment (start 135.35 105.9) (end 137.7 105.9) (width 0.6) (layer "F.Cu") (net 7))
 (segment (start 143.5 105.9) (end 143.5 107.1375) (width 0.6) (layer "F.Cu") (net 7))
 (segment (start 138.944277 105.334792) (end 138.886259 105.334792) (width 0.6) (layer "F.Cu") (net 8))
 (segment (start 141.980285 107.31689) (end 140.6625 108.634675) (width 0.6) (layer "F.Cu") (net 8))
 (segment (start 142.014759 107.02552) (end 141.980285 107.059994) (width 0.6) (layer "F.Cu") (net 8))
 (segment (start 135.35 112.4) (end 135.374 112.376) (width 0.6) (layer "F.Cu") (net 8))
 (segment (start 139.762499 112) (end 140.6625 111.099999) (width 0.6) (layer "F.Cu") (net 8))
 (segment (start 138.451467 104.9) (end 135.4 104.9) (width 0.6) (layer "F.Cu") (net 8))
 (segment (start 141.980285 107.059994) (end 141.980285 107.31689) (width 0.6) (layer "F.Cu") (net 8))
 (segment (start 140.6625 108.634675) (end 140.6625 108.8) (width 0.6) (layer "F.Cu") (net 8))
 (segment (start 135.374 112.376) (end 136.288254 112.376) (width 0.6) (layer "F.Cu") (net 8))
 (segment (start 143.5 108.8625) (end 143.5 111.1375) (width 1) (layer "F.Cu") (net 8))
 (segment (start 135.4 104.9) (end 135.35 104.95) (width 0.6) (layer "F.Cu") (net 8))
 (segment (start 136.288254 112.376) (end 136.664254 112) (width 0.6) (layer "F.Cu") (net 8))
 (segment (start 138.886259 105.334792) (end 138.451467 104.9) (width 0.6) (layer "F.Cu") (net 8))
 (segment (start 140.6625 110) (end 147 110) (width 1) (layer "F.Cu") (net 8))
 (segment (start 140.6625 111.099999) (end 140.6625 110) (width 0.6) (layer "F.Cu") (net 8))
 (segment (start 136.664254 112) (end 139.762499 112) (width 0.6) (layer "F.Cu") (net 8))
 (via (at 142.014759 107.02552) (size 1) (drill 0.5) (layers "F.Cu" "B.Cu") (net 8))
 (via (at 138.944277 105.334792) (size 1) (drill 0.5) (layers "F.Cu" "B.Cu") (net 8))
 (segment (start 138.962891 105.353406) (end 138.944277 105.334792) (width 0.6) (layer "B.Cu") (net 8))
 (segment (start 140.342645 105.353406) (end 138.962891 105.353406) (width 0.6) (layer "B.Cu") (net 8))
 (segment (start 142.014759 107.02552) (end 140.342645 105.353406) (width 0.6) (layer "B.Cu") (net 8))
 (segment (start 118.1375 114.1375) (end 116.1 112.1) (width 1) (layer "F.Cu") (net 9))
 (segment (start 125 112.9125) (end 121.0875 112.9125) (width 1) (layer "F.Cu") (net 9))
 (segment (start 118 114) (end 120 114) (width 1) (layer "F.Cu") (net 9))
 (segment (start 115 113.2) (end 115 114) (width 1) (layer "F.Cu") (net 9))
 (segment (start 117 113) (end 116.1 112.1) (width 1) (layer "F.Cu") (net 9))
 (segment (start 121 113) (end 121 114.1375) (width 1) (layer "F.Cu") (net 9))
 (segment (start 120.0625 109) (end 120.0625 110.161574) (width 1) (layer "F.Cu") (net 9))
 (segment (start 121 114.1375) (end 118.1375 114.1375) (width 1) (layer "F.Cu") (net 9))
 (segment (start 116.1 112.1) (end 115 113.2) (width 1) (layer "F.Cu") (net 9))
 (segment (start 121.0875 112.9125) (end 121 113) (width 1) (layer "F.Cu") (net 9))
 (segment (start 120.0625 110.161574) (end 121 111.099074) (width 1) (layer "F.Cu") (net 9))
 (segment (start 121 113) (end 117 113) (width 1) (layer "F.Cu") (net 9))
 (segment (start 120 114) (end 121 113) (width 1) (layer "F.Cu") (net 9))
 (segment (start 121 111.099074) (end 121 113) (width 1) (layer "F.Cu") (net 9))
 (segment (start 129.9575 105.2625) (end 129.8 105.2625) (width 0.6) (layer "F.Cu") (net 3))
 (segment (start 129.8 105.2625) (end 130.1125 104.95) (width 0.6) (layer "F.Cu") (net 3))
 (segment (start 129.8 105.2625) (end 127.925 105.2625) (width 0.6) (layer "F.Cu") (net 3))
 (segment (start 130.1125 104.95) (end 132.65 104.95) (width 0.6) (layer "F.Cu") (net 3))
 (segment (start 127.925 105.2625) (end 127.8 105.3875) (width 0.6) (layer "F.Cu") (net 3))
 (segment (start 129.9975 105.3025) (end 129.9575 105.2625) (width 0.6) (layer "F.Cu") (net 3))
 (segment (start 133.4325 108.8) (end 133.4325 107.283651) (width 0.6) (layer "F.Cu") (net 5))
 (segment (start 132.998849 106.85) (end 132.65 106.85) (width 0.6) (layer "F.Cu") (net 5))
 (segment (start 133.4325 107.283651) (end 132.998849 106.85) (width 0.6) (layer "F.Cu") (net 5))
 (segment (start 138.3375 108.3375) (end 138.3375 108.8) (width 0.6) (layer "F.Cu") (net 6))
 (segment (start 135.35 106.85) (end 136.85 106.85) (width 0.6) (layer "F.Cu") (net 6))
 (segment (start 134.5675 108.8) (end 134.5675 107.287163) (width 0.6) (layer "F.Cu") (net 6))
 (segment (start 134.5675 107.287163) (end 135.004663 106.85) (width 0.6) (layer "F.Cu") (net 6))
 (segment (start 136.85 106.85) (end 138.3375 108.3375) (width 0.6) (layer "F.Cu") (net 6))
 (segment (start 135.004663 106.85) (end 135.35 106.85) (width 0.6) (layer "F.Cu") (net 6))
 (segment (start 121.45 107.5625) (end 121.9375 108.05) (width 1) (layer "F.Cu") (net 17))
 (segment (start 121.45 105) (end 121.45 107.5625) (width 1) (layer "F.Cu") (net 17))
 (segment (start 123.8625 109.95) (end 125 111.0875) (width 1) (layer "F.Cu") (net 16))
 (segment (start 121.9375 109.95) (end 123.8625 109.95) (width 1) (layer "F.Cu") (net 16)))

